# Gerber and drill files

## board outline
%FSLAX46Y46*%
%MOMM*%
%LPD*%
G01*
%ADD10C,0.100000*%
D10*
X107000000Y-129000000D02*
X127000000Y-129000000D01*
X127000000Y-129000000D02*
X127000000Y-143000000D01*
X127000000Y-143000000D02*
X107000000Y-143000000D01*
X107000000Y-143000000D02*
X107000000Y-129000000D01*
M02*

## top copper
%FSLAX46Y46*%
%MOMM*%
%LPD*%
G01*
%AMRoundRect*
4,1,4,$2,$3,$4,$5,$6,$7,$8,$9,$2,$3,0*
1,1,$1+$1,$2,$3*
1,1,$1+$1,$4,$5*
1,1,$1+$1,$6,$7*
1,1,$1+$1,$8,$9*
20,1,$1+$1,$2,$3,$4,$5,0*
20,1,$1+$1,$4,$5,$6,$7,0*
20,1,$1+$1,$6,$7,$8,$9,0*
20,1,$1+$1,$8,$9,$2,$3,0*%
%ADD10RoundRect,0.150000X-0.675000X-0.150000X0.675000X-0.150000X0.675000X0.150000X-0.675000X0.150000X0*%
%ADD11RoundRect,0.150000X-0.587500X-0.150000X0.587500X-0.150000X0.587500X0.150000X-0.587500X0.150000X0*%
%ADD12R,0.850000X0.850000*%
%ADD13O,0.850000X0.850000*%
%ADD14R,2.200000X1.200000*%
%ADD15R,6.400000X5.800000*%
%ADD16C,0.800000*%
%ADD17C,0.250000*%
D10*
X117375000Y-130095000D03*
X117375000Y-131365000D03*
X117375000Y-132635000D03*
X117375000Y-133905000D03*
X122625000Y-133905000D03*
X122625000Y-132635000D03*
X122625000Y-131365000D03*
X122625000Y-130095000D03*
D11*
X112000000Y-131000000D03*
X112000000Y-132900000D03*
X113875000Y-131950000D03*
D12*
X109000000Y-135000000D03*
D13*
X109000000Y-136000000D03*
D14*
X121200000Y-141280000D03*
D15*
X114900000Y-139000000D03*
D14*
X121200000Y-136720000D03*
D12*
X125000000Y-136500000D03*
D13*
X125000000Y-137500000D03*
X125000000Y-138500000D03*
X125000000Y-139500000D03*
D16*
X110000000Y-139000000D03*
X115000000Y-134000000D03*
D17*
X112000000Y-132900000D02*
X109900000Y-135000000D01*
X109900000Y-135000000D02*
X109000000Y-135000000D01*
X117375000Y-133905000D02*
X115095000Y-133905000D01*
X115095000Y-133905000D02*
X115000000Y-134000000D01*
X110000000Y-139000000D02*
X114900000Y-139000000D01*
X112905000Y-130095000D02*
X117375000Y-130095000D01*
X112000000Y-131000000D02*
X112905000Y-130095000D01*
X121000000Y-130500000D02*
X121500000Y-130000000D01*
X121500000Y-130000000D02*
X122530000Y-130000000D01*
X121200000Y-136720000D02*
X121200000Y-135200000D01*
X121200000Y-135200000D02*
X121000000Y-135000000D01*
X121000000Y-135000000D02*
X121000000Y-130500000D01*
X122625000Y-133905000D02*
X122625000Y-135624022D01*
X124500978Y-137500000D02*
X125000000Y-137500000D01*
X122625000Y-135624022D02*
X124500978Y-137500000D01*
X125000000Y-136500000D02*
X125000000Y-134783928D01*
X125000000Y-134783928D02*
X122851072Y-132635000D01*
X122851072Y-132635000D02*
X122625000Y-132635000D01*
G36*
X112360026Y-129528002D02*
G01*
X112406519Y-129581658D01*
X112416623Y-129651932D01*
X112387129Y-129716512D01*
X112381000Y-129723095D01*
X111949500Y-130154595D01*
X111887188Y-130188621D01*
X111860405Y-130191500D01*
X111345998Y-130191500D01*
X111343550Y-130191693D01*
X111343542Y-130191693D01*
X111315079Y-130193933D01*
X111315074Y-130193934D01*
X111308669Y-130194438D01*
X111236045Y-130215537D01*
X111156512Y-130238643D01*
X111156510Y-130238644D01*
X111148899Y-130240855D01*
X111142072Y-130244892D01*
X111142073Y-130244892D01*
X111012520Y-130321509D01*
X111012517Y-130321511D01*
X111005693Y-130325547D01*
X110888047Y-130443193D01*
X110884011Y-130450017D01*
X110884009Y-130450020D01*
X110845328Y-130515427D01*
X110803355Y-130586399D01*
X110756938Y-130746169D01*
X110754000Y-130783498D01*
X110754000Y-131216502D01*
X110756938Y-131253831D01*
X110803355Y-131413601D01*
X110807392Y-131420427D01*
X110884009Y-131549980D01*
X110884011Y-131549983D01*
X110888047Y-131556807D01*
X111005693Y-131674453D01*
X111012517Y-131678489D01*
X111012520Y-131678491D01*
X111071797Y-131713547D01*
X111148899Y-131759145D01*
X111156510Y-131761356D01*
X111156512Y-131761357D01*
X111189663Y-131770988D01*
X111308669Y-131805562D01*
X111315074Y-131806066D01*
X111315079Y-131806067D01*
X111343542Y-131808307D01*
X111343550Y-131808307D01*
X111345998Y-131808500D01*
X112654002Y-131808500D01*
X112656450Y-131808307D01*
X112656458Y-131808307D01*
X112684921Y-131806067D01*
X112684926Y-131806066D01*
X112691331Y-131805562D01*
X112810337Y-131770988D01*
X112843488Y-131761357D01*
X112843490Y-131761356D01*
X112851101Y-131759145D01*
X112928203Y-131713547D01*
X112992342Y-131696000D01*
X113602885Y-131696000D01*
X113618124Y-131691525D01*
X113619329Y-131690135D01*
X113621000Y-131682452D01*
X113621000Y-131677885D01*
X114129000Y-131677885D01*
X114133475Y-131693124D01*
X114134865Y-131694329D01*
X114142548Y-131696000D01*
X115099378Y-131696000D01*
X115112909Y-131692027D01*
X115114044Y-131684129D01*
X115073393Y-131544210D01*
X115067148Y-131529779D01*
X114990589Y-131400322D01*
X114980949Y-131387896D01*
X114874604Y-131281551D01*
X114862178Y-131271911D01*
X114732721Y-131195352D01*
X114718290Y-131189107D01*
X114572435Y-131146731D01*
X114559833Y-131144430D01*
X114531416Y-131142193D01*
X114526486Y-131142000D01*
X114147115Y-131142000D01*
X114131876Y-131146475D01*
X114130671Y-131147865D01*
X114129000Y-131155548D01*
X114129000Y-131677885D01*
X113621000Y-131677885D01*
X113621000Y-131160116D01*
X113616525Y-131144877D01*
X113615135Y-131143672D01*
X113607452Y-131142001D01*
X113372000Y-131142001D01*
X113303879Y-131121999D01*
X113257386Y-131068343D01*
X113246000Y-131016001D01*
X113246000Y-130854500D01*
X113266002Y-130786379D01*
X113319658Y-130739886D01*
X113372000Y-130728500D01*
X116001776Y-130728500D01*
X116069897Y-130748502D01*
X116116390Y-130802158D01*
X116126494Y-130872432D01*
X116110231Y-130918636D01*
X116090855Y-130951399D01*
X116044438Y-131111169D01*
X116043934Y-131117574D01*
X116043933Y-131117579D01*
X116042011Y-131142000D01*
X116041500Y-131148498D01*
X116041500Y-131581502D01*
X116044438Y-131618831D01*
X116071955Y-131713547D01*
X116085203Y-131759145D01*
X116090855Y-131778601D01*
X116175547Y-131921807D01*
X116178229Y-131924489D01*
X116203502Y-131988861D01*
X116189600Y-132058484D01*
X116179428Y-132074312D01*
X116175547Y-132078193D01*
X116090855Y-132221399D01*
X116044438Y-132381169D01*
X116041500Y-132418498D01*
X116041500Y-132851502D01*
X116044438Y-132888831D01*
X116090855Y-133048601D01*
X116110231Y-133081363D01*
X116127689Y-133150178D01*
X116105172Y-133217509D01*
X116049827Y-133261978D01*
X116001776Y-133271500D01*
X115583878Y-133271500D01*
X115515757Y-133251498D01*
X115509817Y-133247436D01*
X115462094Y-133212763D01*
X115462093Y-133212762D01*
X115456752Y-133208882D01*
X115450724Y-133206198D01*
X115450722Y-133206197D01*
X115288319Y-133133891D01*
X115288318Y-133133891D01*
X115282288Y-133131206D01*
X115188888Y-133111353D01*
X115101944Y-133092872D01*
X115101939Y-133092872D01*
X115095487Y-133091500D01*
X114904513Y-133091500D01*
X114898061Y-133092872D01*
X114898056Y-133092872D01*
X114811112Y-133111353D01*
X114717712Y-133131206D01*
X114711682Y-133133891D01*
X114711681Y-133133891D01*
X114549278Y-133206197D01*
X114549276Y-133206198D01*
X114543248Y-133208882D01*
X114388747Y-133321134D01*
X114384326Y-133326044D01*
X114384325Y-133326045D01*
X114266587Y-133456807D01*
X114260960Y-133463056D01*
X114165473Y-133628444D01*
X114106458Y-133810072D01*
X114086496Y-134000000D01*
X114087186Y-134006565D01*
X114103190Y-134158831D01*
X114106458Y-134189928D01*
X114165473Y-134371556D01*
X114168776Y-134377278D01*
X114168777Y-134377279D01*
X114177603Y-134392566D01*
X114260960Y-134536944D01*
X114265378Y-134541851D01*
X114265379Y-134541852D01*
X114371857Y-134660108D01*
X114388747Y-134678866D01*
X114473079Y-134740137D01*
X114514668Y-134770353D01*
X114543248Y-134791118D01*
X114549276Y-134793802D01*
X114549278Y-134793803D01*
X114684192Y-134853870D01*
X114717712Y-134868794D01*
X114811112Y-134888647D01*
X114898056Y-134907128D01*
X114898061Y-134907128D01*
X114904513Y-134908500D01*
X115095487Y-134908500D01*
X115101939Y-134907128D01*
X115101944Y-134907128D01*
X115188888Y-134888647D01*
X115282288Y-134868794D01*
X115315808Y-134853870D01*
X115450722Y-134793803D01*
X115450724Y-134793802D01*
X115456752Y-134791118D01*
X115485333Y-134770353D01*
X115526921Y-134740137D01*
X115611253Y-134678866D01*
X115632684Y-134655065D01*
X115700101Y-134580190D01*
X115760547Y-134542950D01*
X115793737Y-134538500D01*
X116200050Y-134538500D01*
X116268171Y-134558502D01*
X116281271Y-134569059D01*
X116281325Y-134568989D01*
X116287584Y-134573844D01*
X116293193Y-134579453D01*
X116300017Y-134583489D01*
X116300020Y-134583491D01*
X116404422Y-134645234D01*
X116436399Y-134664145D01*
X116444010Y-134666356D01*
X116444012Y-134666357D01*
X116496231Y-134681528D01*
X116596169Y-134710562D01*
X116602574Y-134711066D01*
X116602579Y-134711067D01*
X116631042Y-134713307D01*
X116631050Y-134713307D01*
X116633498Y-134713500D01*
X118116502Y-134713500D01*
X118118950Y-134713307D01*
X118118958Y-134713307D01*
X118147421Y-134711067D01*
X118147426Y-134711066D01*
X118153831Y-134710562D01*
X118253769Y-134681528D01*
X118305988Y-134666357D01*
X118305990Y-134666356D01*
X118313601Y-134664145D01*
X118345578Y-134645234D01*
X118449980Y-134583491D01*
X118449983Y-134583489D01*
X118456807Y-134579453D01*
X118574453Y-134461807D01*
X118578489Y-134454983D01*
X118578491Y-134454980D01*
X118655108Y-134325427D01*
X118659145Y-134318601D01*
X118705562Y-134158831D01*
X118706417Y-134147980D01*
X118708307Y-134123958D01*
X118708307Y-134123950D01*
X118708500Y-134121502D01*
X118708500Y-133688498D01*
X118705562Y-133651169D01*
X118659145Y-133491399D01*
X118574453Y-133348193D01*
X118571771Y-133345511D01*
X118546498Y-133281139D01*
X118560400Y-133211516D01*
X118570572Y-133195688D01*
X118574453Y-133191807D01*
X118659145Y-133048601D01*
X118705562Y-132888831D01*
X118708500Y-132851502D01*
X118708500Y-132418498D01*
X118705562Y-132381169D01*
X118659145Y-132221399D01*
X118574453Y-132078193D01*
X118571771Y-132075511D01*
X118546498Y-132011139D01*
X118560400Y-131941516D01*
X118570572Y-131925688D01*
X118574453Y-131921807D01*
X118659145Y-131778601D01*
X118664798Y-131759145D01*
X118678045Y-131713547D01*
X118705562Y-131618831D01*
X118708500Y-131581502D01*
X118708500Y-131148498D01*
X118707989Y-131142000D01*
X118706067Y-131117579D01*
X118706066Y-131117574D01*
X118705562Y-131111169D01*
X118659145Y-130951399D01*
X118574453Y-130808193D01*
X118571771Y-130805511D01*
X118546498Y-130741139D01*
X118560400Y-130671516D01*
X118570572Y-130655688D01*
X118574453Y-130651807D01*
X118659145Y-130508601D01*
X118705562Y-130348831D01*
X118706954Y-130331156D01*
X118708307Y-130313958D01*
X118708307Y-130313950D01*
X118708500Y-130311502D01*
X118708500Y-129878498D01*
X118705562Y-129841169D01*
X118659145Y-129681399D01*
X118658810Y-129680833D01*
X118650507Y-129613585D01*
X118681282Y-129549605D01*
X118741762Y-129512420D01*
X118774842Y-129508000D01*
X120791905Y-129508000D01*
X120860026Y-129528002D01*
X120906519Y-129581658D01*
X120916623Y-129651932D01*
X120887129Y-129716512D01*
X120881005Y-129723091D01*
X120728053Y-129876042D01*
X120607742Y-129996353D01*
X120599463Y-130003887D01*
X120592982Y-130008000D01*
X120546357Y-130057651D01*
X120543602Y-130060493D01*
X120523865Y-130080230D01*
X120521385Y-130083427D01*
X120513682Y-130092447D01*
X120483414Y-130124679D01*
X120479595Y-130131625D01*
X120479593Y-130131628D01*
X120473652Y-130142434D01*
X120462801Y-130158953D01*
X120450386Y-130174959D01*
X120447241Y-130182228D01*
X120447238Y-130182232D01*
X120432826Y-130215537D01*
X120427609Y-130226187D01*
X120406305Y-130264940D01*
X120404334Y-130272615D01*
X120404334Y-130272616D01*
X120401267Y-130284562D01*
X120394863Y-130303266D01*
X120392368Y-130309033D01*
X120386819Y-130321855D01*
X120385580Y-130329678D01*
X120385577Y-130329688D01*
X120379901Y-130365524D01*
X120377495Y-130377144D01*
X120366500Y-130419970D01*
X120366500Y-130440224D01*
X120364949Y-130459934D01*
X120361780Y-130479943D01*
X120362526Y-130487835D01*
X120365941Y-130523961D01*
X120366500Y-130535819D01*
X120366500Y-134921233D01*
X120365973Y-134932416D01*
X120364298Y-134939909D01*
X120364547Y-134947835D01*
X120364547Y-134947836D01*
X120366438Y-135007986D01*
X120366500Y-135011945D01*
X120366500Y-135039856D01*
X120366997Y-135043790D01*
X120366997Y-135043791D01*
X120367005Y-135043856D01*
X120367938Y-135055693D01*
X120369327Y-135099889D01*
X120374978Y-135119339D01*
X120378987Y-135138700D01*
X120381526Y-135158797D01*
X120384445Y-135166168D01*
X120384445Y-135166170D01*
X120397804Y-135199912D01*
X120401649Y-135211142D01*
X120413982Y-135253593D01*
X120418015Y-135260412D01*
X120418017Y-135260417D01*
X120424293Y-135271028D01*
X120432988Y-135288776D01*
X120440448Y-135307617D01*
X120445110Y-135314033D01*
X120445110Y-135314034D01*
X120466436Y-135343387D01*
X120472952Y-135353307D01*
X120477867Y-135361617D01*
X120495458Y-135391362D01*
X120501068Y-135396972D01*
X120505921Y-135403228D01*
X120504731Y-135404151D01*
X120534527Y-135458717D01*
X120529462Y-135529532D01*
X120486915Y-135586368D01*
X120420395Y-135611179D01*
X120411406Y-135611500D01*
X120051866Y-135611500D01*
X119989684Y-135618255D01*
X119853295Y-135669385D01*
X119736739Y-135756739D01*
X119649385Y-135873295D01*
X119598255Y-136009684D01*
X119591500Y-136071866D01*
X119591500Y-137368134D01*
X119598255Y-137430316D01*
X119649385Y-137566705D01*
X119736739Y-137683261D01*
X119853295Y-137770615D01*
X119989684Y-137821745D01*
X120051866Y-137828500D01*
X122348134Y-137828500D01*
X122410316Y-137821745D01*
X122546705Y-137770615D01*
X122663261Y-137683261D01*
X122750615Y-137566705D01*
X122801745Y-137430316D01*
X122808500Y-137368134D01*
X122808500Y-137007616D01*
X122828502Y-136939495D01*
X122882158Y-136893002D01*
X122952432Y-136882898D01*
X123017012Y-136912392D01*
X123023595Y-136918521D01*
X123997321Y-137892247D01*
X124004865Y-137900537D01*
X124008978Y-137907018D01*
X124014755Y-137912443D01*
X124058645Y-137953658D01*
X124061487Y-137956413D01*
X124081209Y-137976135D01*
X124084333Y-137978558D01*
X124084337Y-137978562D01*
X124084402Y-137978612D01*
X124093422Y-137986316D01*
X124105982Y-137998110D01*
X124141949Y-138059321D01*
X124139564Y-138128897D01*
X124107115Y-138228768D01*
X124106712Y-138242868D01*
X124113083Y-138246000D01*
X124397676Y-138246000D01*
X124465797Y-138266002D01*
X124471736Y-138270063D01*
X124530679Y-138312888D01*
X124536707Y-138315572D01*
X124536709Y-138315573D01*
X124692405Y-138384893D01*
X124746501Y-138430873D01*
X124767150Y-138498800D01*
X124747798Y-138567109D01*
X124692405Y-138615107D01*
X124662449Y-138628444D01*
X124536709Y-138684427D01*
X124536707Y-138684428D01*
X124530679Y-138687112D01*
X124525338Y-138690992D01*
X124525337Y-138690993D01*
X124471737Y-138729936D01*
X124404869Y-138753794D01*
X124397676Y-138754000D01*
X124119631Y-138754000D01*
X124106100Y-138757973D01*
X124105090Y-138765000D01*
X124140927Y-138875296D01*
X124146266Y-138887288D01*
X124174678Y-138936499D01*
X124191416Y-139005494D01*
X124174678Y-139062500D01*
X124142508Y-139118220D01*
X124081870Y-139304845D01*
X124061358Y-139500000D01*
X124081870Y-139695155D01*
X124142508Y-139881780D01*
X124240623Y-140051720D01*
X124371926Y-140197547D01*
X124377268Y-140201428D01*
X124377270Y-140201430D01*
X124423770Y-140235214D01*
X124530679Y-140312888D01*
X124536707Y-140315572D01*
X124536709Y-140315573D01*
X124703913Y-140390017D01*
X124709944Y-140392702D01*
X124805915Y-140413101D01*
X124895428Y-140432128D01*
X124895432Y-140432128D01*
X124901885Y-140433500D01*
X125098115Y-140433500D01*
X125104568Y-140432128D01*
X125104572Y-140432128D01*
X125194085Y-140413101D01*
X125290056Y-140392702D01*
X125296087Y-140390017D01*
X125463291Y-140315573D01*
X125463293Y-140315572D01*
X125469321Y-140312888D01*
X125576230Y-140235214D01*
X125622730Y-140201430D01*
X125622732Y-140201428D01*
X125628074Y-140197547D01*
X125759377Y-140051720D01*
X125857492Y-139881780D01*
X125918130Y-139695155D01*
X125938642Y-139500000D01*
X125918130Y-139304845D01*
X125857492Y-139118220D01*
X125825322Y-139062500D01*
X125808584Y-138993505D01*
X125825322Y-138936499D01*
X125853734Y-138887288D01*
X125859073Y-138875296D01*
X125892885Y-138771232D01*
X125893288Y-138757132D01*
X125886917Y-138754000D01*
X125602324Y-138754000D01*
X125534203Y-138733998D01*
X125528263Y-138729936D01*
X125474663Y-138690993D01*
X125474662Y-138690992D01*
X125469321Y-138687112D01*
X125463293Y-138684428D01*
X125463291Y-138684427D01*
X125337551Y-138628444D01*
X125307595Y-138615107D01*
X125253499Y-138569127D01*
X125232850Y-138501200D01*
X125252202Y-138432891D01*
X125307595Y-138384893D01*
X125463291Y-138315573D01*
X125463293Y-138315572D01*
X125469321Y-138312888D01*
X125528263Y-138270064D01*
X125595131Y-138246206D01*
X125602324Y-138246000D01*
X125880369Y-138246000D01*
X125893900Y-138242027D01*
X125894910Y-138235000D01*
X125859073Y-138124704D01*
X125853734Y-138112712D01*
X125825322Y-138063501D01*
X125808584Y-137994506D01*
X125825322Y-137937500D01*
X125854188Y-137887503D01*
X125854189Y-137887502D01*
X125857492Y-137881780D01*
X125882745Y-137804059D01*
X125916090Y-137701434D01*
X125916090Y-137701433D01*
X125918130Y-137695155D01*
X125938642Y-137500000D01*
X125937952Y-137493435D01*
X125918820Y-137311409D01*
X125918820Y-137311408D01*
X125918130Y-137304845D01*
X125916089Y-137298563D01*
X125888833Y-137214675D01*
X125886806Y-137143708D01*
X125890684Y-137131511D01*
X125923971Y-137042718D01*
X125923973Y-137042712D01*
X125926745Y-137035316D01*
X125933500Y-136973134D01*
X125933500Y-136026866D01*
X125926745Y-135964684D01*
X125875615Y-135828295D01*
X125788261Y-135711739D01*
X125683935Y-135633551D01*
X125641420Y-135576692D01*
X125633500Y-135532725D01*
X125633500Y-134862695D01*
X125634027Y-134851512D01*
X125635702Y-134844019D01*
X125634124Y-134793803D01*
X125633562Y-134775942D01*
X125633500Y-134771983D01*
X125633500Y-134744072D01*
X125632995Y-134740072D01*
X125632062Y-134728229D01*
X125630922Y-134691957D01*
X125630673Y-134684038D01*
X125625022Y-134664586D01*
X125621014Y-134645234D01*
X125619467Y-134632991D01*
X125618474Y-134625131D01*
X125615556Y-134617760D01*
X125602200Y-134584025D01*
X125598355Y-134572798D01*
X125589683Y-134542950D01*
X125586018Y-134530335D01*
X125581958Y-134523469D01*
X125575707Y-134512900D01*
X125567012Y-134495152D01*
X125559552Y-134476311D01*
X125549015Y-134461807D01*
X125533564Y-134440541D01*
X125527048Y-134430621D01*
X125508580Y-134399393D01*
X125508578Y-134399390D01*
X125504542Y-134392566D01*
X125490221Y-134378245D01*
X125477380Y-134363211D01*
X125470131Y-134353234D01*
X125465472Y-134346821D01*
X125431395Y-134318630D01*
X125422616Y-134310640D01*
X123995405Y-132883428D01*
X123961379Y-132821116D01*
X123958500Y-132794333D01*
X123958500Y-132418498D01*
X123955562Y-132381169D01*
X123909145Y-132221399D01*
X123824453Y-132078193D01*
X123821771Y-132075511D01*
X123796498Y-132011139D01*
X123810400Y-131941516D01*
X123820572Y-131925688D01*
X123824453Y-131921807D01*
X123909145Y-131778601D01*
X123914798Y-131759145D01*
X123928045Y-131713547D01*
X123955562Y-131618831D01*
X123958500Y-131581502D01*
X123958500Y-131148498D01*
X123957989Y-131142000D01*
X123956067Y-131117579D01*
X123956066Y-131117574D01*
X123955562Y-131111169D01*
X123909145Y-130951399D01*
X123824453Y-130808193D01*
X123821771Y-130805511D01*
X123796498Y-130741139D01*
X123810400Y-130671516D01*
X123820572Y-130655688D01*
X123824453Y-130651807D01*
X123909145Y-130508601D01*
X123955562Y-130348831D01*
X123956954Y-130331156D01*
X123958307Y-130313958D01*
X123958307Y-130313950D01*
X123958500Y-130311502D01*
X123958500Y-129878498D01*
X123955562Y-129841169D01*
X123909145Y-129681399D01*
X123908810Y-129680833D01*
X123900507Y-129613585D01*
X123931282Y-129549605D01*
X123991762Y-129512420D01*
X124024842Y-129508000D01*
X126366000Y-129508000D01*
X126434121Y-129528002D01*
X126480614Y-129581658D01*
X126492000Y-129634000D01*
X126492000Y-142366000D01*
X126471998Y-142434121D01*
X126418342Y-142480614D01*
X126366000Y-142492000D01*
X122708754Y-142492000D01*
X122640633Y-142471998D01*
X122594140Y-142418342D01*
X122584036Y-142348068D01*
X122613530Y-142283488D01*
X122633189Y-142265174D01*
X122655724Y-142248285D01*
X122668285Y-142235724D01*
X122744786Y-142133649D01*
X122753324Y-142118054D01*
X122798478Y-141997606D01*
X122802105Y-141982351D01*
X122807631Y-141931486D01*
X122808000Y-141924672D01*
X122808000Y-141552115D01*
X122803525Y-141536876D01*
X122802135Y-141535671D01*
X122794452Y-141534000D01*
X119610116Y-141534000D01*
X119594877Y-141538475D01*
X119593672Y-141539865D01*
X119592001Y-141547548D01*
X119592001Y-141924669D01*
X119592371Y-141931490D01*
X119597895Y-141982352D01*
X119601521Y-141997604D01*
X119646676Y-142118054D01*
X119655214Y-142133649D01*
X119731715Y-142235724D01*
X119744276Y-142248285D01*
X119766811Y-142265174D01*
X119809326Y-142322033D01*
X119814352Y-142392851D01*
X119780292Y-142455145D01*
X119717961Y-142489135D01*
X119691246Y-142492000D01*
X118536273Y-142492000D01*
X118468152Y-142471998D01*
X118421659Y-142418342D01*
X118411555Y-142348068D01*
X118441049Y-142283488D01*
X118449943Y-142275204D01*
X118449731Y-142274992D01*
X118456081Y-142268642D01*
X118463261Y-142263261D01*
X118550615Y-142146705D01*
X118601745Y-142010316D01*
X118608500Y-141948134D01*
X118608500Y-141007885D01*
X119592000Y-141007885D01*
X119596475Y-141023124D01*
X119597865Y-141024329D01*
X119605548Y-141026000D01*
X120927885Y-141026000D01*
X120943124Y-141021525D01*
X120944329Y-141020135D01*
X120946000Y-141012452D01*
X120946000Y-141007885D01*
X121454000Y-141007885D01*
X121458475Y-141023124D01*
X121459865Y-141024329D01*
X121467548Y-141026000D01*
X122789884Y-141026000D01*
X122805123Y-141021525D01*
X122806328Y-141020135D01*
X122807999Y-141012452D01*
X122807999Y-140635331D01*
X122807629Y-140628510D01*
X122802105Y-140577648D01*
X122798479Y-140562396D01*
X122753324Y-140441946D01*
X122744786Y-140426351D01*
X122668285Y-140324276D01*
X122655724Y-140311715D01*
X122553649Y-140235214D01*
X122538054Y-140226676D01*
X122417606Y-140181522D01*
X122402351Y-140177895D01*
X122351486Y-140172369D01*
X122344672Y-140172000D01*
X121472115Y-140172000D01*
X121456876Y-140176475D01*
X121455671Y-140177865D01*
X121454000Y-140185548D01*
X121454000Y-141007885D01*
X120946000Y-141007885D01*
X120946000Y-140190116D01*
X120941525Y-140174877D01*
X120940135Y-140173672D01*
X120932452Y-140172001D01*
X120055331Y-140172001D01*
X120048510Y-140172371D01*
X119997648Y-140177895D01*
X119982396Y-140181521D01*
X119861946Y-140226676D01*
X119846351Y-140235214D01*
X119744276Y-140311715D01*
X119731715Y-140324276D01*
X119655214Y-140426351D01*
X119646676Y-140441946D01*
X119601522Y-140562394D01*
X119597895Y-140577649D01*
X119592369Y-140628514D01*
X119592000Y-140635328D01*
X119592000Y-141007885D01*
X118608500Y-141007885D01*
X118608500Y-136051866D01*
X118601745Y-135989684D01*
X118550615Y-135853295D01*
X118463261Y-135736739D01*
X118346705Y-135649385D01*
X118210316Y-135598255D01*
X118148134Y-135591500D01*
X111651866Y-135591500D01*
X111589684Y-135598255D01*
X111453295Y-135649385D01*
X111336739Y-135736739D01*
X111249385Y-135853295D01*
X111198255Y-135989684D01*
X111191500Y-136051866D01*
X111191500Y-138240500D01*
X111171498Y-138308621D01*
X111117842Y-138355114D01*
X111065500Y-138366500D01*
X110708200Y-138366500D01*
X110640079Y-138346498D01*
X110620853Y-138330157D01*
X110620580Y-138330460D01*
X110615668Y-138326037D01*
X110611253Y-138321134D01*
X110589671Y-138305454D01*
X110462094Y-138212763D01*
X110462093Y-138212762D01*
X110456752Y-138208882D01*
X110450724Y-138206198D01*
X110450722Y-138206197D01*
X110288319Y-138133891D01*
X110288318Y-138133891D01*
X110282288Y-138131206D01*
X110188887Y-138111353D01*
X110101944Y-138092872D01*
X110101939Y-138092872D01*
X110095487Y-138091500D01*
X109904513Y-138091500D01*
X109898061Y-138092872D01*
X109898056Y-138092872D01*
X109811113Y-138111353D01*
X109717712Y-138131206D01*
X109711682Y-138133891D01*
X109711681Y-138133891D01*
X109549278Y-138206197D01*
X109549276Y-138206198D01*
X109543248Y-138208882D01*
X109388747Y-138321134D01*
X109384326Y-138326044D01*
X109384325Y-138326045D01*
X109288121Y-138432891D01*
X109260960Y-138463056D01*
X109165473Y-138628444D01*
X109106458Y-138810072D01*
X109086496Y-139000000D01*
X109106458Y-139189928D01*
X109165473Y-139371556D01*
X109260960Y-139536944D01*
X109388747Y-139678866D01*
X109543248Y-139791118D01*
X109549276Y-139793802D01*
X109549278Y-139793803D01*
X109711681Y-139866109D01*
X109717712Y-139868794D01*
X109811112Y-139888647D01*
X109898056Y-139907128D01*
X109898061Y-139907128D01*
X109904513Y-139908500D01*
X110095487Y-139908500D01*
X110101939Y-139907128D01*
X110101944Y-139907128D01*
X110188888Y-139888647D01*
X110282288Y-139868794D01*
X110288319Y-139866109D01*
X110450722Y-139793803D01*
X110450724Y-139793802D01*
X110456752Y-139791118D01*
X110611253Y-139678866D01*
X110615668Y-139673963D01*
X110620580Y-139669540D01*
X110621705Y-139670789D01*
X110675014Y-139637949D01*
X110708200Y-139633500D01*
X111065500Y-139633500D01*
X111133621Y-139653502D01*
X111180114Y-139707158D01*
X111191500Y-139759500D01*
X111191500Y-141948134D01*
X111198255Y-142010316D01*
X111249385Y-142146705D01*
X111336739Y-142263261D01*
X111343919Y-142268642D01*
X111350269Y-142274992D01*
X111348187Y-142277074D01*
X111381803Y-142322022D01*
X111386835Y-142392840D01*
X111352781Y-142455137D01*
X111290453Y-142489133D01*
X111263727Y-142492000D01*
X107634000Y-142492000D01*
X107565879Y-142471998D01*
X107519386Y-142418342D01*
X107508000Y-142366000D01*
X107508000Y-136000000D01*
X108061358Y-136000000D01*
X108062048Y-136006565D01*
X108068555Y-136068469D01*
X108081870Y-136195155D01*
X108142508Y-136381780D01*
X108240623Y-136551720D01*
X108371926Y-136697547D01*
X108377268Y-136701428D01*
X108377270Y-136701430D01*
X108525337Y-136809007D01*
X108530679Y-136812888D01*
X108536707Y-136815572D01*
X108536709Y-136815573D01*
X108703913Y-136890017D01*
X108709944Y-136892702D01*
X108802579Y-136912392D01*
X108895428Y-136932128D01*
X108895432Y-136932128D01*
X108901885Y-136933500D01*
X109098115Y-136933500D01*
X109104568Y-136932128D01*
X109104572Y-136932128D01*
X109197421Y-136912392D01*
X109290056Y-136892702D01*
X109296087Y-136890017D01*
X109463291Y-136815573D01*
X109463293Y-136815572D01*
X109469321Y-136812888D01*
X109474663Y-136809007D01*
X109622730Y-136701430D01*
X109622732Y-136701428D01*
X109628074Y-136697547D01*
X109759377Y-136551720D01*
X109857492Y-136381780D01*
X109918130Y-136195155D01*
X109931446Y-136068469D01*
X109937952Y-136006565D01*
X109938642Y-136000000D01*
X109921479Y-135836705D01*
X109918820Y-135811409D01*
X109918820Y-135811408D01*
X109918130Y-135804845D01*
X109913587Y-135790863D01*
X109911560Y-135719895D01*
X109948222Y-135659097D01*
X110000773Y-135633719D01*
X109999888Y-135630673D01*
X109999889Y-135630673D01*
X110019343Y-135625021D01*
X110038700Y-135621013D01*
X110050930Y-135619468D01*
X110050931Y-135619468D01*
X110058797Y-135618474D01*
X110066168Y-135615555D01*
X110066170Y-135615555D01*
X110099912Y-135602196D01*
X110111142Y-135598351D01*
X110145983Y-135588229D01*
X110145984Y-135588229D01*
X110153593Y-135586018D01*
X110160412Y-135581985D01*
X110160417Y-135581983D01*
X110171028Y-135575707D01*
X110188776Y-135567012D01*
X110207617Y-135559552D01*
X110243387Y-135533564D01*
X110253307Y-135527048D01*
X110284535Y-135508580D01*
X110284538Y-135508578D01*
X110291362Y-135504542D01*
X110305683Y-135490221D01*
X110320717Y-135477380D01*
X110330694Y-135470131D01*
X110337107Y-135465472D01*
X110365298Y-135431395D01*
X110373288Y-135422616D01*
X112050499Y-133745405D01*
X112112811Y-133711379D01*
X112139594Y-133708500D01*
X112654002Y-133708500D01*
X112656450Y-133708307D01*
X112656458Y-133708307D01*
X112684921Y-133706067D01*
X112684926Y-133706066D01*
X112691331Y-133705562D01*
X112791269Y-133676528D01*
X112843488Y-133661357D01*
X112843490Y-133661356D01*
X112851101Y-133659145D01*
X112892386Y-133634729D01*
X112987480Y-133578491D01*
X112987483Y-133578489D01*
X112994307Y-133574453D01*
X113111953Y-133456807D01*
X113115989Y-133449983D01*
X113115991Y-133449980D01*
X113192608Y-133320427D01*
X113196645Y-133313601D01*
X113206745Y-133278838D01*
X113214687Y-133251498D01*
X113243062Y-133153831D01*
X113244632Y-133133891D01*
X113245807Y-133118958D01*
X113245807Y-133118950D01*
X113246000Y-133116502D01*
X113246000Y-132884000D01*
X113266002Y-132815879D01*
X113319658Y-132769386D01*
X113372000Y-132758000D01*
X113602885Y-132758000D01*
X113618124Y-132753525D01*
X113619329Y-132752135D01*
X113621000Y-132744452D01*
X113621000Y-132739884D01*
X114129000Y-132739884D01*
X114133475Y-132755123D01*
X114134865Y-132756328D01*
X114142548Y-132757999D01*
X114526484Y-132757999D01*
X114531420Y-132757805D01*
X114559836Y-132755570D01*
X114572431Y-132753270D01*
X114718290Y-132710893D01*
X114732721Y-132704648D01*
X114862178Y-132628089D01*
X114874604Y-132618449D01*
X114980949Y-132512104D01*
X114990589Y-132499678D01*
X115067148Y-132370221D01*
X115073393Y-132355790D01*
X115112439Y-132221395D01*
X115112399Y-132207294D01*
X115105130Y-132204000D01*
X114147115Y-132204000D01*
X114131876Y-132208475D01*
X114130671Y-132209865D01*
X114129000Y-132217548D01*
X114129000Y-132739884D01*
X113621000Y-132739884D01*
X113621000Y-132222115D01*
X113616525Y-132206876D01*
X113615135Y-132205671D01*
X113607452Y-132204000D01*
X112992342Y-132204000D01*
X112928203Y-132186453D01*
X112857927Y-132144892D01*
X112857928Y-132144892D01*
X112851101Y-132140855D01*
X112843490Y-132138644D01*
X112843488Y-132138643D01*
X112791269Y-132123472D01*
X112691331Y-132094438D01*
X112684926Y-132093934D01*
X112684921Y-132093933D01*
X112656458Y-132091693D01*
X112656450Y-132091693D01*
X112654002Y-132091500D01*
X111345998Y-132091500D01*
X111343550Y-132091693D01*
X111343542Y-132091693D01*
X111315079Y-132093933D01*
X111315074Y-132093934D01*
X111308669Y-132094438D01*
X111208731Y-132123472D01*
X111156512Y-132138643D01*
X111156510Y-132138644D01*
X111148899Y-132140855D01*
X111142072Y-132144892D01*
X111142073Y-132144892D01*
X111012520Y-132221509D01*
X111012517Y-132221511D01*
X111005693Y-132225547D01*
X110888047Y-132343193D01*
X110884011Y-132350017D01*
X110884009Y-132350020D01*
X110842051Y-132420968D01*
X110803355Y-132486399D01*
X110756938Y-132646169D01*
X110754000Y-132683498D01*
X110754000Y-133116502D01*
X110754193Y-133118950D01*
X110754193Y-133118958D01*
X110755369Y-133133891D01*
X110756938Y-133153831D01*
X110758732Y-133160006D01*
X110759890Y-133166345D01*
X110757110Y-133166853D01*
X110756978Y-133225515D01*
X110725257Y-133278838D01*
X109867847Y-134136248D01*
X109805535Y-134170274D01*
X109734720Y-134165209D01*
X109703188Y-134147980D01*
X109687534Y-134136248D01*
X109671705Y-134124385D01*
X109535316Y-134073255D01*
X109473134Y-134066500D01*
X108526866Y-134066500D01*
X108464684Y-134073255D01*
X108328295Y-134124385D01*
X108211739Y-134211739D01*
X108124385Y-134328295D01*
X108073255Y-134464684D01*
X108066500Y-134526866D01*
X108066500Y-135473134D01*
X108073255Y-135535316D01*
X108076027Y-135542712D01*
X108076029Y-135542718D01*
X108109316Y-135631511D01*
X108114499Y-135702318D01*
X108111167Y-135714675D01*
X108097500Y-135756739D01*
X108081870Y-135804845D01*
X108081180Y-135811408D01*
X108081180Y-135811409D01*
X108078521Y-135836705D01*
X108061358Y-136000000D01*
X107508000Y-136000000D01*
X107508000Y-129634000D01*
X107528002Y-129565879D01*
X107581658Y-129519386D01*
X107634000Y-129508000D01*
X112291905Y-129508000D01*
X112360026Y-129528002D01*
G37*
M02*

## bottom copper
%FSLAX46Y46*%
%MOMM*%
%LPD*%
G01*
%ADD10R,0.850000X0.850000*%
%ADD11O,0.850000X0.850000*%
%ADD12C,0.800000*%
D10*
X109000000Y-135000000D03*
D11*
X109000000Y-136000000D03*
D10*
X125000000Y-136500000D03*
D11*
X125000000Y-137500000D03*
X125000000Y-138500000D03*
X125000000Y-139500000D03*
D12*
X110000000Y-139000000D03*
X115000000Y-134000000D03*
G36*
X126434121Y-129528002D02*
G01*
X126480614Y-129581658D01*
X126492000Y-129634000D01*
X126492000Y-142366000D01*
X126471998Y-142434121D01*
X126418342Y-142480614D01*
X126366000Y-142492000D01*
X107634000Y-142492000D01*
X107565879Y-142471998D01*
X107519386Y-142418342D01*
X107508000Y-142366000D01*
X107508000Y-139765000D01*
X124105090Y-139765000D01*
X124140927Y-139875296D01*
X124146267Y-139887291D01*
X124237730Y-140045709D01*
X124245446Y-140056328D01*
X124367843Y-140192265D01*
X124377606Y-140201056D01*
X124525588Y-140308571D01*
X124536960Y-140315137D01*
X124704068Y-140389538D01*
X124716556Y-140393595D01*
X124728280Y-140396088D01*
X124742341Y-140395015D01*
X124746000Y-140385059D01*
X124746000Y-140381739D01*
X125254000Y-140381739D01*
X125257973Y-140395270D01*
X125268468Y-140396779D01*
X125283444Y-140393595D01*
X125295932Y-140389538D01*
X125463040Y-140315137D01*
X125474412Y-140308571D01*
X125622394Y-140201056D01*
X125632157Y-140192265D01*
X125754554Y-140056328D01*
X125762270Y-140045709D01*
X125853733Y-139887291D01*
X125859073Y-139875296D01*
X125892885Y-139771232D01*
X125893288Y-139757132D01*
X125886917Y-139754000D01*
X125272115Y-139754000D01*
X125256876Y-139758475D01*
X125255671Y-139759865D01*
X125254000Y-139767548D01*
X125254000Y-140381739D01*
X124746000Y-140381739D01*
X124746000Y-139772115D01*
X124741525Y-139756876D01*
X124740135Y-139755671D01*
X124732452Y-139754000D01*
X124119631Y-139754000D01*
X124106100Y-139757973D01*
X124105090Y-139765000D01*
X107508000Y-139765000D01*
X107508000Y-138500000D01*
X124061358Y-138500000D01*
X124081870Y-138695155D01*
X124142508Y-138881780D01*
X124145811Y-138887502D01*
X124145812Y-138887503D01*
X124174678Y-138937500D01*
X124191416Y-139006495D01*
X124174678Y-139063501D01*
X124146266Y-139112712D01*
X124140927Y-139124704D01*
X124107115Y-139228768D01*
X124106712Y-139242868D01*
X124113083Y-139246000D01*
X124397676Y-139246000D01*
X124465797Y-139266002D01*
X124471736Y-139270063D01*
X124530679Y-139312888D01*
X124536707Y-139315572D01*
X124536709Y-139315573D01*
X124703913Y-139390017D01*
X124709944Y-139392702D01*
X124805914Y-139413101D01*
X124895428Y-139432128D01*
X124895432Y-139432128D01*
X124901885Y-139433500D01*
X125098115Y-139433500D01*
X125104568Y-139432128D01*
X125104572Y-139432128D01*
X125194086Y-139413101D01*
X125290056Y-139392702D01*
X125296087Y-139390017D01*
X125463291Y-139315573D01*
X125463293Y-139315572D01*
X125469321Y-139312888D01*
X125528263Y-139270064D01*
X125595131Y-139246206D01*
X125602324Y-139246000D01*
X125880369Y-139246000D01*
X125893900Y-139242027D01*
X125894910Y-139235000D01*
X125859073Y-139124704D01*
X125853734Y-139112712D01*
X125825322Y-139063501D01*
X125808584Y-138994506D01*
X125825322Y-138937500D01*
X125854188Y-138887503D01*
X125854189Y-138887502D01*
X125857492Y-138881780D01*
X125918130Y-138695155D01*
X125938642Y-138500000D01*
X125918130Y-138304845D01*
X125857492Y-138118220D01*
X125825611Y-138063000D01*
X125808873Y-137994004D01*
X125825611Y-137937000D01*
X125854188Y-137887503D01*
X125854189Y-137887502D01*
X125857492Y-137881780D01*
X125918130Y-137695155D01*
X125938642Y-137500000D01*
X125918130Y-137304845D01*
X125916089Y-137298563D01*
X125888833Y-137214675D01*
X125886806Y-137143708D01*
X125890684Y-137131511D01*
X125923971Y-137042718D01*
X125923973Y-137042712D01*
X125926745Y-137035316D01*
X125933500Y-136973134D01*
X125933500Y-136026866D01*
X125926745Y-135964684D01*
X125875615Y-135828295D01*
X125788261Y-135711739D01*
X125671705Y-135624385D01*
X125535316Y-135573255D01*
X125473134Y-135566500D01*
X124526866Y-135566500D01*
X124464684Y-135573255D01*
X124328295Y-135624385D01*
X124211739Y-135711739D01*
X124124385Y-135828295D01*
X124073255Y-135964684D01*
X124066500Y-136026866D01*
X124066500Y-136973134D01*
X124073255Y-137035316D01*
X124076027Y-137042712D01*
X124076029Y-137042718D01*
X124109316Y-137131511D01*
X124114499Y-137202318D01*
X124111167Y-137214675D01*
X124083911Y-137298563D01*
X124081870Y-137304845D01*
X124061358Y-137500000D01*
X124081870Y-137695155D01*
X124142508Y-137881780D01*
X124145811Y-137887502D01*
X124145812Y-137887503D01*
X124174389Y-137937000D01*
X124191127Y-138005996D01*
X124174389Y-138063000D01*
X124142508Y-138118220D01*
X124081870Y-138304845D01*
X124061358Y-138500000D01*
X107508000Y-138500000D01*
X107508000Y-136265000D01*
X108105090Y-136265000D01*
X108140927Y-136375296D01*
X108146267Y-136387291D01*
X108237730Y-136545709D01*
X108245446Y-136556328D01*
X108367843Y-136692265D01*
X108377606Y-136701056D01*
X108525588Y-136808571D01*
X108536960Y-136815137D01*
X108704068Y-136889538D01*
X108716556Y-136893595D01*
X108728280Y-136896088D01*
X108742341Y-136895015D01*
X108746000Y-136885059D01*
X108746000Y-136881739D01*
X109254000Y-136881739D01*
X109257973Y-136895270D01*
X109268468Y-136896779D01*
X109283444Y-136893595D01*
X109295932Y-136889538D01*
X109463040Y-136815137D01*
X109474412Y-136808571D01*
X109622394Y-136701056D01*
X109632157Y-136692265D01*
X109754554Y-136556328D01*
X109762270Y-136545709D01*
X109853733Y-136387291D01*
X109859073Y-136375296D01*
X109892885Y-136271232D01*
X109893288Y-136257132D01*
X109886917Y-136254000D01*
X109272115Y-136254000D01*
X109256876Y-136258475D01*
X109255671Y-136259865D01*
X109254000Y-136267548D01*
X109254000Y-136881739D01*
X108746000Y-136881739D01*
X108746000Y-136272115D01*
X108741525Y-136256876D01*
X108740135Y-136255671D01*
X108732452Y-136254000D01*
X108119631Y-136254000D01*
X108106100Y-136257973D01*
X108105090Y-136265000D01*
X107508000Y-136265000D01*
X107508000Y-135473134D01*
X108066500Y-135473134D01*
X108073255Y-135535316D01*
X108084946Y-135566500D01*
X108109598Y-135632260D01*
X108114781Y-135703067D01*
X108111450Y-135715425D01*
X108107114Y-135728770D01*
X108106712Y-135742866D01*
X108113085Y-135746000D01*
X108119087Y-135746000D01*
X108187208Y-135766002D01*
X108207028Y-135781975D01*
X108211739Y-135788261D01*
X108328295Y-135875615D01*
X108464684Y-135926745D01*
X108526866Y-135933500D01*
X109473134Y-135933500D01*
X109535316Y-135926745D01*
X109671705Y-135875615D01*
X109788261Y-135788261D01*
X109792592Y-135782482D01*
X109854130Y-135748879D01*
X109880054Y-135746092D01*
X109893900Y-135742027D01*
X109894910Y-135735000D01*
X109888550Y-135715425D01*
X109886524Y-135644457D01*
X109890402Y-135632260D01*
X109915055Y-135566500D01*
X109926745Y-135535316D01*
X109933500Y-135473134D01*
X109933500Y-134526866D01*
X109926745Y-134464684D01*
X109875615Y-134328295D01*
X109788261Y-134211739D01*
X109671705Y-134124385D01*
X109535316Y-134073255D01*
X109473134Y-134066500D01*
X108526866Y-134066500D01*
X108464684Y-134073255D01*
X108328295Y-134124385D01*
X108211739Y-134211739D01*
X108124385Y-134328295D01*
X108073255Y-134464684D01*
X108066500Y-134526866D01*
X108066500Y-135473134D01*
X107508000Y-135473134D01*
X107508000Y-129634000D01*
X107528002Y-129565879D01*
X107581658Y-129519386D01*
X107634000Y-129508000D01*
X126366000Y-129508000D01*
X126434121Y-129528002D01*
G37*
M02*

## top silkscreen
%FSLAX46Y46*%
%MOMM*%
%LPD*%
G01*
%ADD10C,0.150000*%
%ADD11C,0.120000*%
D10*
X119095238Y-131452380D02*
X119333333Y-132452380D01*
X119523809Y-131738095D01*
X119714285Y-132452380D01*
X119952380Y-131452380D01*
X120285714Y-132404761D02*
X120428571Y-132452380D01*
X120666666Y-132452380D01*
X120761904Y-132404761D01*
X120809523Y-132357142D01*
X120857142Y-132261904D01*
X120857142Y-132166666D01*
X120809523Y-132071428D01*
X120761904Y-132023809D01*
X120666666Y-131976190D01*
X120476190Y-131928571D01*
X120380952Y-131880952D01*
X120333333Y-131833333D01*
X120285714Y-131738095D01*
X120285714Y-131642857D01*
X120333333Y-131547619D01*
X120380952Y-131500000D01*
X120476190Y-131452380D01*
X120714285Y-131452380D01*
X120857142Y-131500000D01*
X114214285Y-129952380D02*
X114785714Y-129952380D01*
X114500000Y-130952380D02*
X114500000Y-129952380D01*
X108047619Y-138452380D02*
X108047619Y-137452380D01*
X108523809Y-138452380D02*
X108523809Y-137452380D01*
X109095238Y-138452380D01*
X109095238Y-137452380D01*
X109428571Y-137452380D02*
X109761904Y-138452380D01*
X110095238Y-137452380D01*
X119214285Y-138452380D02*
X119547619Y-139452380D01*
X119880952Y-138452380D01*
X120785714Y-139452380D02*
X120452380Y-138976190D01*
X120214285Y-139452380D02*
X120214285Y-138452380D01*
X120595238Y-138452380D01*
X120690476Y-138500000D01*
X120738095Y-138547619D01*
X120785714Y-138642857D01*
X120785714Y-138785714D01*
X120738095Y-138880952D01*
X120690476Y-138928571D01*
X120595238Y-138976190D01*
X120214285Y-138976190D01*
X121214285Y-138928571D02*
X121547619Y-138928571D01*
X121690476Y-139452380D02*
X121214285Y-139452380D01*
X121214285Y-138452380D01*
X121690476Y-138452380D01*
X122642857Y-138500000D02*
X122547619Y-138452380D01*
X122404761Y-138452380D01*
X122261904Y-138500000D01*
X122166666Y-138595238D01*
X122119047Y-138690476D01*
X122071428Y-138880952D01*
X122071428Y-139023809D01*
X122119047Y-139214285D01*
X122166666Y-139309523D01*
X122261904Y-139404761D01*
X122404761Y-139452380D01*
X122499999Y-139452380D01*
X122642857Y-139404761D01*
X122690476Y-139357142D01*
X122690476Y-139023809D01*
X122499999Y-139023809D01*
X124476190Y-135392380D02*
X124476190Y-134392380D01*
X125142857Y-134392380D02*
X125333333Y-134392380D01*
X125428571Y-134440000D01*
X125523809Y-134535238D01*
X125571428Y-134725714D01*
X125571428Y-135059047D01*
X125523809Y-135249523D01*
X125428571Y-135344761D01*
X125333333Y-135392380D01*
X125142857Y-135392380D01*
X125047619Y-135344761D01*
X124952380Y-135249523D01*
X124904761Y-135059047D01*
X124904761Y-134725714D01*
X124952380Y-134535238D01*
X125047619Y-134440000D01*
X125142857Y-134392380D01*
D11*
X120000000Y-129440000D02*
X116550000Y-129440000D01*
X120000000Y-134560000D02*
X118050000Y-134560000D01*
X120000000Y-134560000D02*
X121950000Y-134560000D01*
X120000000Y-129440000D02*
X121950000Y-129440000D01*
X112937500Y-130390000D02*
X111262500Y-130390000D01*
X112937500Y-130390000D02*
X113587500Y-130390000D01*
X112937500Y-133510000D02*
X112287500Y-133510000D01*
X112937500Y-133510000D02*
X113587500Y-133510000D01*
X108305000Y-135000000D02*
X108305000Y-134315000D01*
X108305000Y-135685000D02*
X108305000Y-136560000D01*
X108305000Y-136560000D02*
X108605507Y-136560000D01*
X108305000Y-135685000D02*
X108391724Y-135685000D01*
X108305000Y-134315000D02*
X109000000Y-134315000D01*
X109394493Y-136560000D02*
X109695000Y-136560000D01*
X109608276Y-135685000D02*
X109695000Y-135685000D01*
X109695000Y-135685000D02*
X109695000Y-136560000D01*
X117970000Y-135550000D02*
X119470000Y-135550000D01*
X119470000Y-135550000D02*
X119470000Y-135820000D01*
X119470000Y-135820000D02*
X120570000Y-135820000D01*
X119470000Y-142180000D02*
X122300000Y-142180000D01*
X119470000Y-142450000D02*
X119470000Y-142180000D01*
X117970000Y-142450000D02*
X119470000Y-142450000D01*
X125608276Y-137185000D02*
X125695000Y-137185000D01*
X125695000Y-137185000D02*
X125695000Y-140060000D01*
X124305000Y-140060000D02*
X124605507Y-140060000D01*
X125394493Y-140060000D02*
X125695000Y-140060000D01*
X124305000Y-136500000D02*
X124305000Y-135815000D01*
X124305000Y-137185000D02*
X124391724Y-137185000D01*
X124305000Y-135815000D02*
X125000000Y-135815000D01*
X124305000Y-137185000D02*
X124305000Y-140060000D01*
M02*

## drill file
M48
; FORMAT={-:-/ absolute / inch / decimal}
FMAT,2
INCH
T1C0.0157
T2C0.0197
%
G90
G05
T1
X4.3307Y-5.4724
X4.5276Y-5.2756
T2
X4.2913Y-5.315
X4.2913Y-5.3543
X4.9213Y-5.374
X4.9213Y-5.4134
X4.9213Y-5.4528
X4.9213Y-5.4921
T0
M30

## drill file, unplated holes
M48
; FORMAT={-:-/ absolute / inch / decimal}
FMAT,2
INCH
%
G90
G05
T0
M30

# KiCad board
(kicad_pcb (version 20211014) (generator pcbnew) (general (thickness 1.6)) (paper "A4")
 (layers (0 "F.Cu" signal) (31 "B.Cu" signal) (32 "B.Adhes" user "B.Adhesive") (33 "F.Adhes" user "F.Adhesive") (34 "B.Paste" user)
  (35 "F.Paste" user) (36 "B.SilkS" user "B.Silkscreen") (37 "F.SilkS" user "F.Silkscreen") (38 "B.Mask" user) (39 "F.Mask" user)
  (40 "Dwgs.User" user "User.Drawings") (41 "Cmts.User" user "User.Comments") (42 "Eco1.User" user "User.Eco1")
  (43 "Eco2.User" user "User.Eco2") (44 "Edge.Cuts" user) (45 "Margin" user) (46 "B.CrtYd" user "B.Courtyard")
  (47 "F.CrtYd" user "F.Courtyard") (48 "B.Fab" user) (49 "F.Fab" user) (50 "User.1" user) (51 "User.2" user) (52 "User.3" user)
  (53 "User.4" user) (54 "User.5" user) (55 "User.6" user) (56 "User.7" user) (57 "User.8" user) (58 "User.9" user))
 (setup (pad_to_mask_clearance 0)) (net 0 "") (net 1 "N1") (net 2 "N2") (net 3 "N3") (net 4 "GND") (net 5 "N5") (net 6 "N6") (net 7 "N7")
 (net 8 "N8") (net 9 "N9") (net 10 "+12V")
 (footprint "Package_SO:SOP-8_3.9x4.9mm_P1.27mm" (layer "F.Cu") (at 120 132)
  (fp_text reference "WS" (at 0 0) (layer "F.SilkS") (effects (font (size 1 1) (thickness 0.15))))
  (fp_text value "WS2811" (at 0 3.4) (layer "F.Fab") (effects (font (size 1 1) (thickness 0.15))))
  (fp_line (start 0 -2.56) (end -3.45 -2.56) (layer "F.SilkS") (width 0.12))
  (fp_line (start 0 2.56) (end -1.95 2.56) (layer "F.SilkS") (width 0.12))
  (fp_line (start 0 2.56) (end 1.95 2.56) (layer "F.SilkS") (width 0.12))
  (fp_line (start 0 -2.56) (end 1.95 -2.56) (layer "F.SilkS") (width 0.12))
  (pad "1" smd roundrect (at -2.625 -1.905) (size 1.65 0.6) (layers "F.Cu" "F.Paste" "F.Mask") (roundrect_rratio 0.25) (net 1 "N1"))
  (pad "2" smd roundrect (at -2.625 -0.635) (size 1.65 0.6) (layers "F.Cu" "F.Paste" "F.Mask") (roundrect_rratio 0.25) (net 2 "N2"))
  (pad "3" smd roundrect (at -2.625 0.635) (size 1.65 0.6) (layers "F.Cu" "F.Paste" "F.Mask") (roundrect_rratio 0.25) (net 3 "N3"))
  (pad "4" smd roundrect (at -2.625 1.905) (size 1.65 0.6) (layers "F.Cu" "F.Paste" "F.Mask") (roundrect_rratio 0.25) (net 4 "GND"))
  (pad "5" smd roundrect (at 2.625 1.905) (size 1.65 0.6) (layers "F.Cu" "F.Paste" "F.Mask") (roundrect_rratio 0.25) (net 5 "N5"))
  (pad "6" smd roundrect (at 2.625 0.635) (size 1.65 0.6) (layers "F.Cu" "F.Paste" "F.Mask") (roundrect_rratio 0.25) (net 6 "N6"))
  (pad "7" smd roundrect (at 2.625 -0.635) (size 1.65 0.6) (layers "F.Cu" "F.Paste" "F.Mask") (roundrect_rratio 0.25) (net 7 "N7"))
  (pad "8" smd roundrect (at 2.625 -1.905) (size 1.65 0.6) (layers "F.Cu" "F.Paste" "F.Mask") (roundrect_rratio 0.25) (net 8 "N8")))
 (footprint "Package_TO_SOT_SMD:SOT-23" (layer "F.Cu") (at 112.9375 131.95)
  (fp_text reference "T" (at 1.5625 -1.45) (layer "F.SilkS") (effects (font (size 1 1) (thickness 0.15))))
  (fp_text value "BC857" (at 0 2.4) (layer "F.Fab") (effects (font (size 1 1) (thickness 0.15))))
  (fp_line (start 0 -1.56) (end -1.675 -1.56) (layer "F.SilkS") (width 0.12))
  (fp_line (start 0 -1.56) (end 0.65 -1.56) (layer "F.SilkS") (width 0.12))
  (fp_line (start 0 1.56) (end -0.65 1.56) (layer "F.SilkS") (width 0.12))
  (fp_line (start 0 1.56) (end 0.65 1.56) (layer "F.SilkS") (width 0.12))
  (pad "1" smd roundrect (at -0.9375 -0.95) (size 1.475 0.6) (layers "F.Cu" "F.Paste" "F.Mask") (roundrect_rratio 0.25) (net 1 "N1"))
  (pad "2" smd roundrect (at -0.9375 0.95) (size 1.475 0.6) (layers "F.Cu" "F.Paste" "F.Mask") (roundrect_rratio 0.25) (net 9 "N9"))
  (pad "3" smd roundrect (at 0.9375 0) (size 1.475 0.6) (layers "F.Cu" "F.Paste" "F.Mask") (roundrect_rratio 0.25) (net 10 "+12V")))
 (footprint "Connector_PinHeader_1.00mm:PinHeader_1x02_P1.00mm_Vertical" (layer "F.Cu") (at 109 135)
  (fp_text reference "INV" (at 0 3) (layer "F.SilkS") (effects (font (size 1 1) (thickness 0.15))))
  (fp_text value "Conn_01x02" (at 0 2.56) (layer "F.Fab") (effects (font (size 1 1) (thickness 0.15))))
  (fp_line (start -0.695 0) (end -0.695 -0.685) (layer "F.SilkS") (width 0.12))
  (fp_line (start -0.695 0.685) (end -0.695 1.56) (layer "F.SilkS") (width 0.12))
  (fp_line (start -0.695 1.56) (end -0.394493 1.56) (layer "F.SilkS") (width 0.12))
  (fp_line (start -0.695 0.685) (end -0.608276 0.685) (layer "F.SilkS") (width 0.12))
  (fp_line (start -0.695 -0.685) (end 0 -0.685) (layer "F.SilkS") (width 0.12))
  (fp_line (start 0.394493 1.56) (end 0.695 1.56) (layer "F.SilkS") (width 0.12))
  (fp_line (start 0.608276 0.685) (end 0.695 0.685) (layer "F.SilkS") (width 0.12))
  (fp_line (start 0.695 0.685) (end 0.695 1.56) (layer "F.SilkS") (width 0.12))
  (pad "1" thru_hole rect (at 0 0) (size 0.85 0.85) (drill 0.5) (layers *.Cu *.Mask) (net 9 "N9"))
  (pad "2" thru_hole oval (at 0 1) (size 0.85 0.85) (drill 0.5) (layers *.Cu *.Mask) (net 4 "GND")))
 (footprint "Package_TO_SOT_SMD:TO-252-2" (layer "F.Cu") (at 117 139 180)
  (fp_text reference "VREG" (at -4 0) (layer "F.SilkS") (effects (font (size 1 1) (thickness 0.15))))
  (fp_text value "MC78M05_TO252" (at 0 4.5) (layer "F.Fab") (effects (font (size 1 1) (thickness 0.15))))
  (fp_line (start -0.97 3.45) (end -2.47 3.45) (layer "F.SilkS") (width 0.12))
  (fp_line (start -2.47 3.45) (end -2.47 3.18) (layer "F.SilkS") (width 0.12))
  (fp_line (start -2.47 3.18) (end -3.57 3.18) (layer "F.SilkS") (width 0.12))
  (fp_line (start -2.47 -3.18) (end -5.3 -3.18) (layer "F.SilkS") (width 0.12))
  (fp_line (start -2.47 -3.45) (end -2.47 -3.18) (layer "F.SilkS") (width 0.12))
  (fp_line (start -0.97 -3.45) (end -2.47 -3.45) (layer "F.SilkS") (width 0.12))
  (pad "" smd rect (at 0.425 -1.525 180) (size 3.05 2.75) (layers "F.Paste"))
  (pad "" smd rect (at 3.775 1.525 180) (size 3.05 2.75) (layers "F.Paste"))
  (pad "" smd rect (at 3.775 -1.525 180) (size 3.05 2.75) (layers "F.Paste"))
  (pad "" smd rect (at 0.425 1.525 180) (size 3.05 2.75) (layers "F.Paste"))
  (pad "1" smd rect (at -4.2 -2.28 180) (size 2.2 1.2) (layers "F.Cu" "F.Paste" "F.Mask") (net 10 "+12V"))
  (pad "2" smd rect (at 2.1 0 180) (size 6.4 5.8) (layers "F.Cu" "F.Mask") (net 4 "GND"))
  (pad "3" smd rect (at -4.2 2.28 180) (size 2.2 1.2) (layers "F.Cu" "F.Paste" "F.Mask") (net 8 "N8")))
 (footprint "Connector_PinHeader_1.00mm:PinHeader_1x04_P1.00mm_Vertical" (layer "F.Cu") (at 125 136.5)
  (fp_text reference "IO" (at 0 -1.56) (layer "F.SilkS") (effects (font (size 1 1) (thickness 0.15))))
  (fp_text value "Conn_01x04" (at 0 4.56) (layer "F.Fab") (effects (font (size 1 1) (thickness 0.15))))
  (fp_line (start 0.608276 0.685) (end 0.695 0.685) (layer "F.SilkS") (width 0.12))
  (fp_line (start 0.695 0.685) (end 0.695 3.56) (layer "F.SilkS") (width 0.12))
  (fp_line (start -0.695 3.56) (end -0.394493 3.56) (layer "F.SilkS") (width 0.12))
  (fp_line (start 0.394493 3.56) (end 0.695 3.56) (layer "F.SilkS") (width 0.12))
  (fp_line (start -0.695 0) (end -0.695 -0.685) (layer "F.SilkS") (width 0.12))
  (fp_line (start -0.695 0.685) (end -0.608276 0.685) (layer "F.SilkS") (width 0.12))
  (fp_line (start -0.695 -0.685) (end 0 -0.685) (layer "F.SilkS") (width 0.12))
  (fp_line (start -0.695 0.685) (end -0.695 3.56) (layer "F.SilkS") (width 0.12))
  (pad "1" thru_hole rect (at 0 0) (size 0.85 0.85) (drill 0.5) (layers *.Cu *.Mask) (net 6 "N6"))
  (pad "2" thru_hole oval (at 0 1) (size 0.85 0.85) (drill 0.5) (layers *.Cu *.Mask) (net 5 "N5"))
  (pad "3" thru_hole oval (at 0 2) (size 0.85 0.85) (drill 0.5) (layers *.Cu *.Mask) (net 10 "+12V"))
  (pad "4" thru_hole oval (at 0 3) (size 0.85 0.85) (drill 0.5) (layers *.Cu *.Mask) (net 4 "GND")))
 (gr_rect (start 107 129) (end 127 143) (layer "Edge.Cuts") (width 0.1) (fill none))
 (segment (start 109.9 135) (end 109 135) (width 0.25) (layer "F.Cu") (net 9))
 (segment (start 112 132.9) (end 109.9 135) (width 0.25) (layer "F.Cu") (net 9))
 (segment (start 117.375 133.905) (end 115.095 133.905) (width 0.25) (layer "F.Cu") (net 4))
 (segment (start 110 139) (end 114.9 139) (width 0.25) (layer "F.Cu") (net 4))
 (segment (start 115.095 133.905) (end 115 134) (width 0.25) (layer "F.Cu") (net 4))
 (via (at 110 139) (size 0.8) (drill 0.4) (layers "F.Cu" "B.Cu") (free) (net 4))
 (via (at 115 134) (size 0.8) (drill 0.4) (layers "F.Cu" "B.Cu") (free) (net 4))
 (segment (start 112.905 130.095) (end 117.375 130.095) (width 0.25) (layer "F.Cu") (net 1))
 (segment (start 112 131) (end 112.905 130.095) (width 0.25) (layer "F.Cu") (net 1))
 (segment (start 121 130.5) (end 121.5 130) (width 0.25) (layer "F.Cu") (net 8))
 (segment (start 121.5 130) (end 122.53 130) (width 0.25) (layer "F.Cu") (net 8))
 (segment (start 121.2 136.72) (end 121.2 135.2) (width 0.25) (layer "F.Cu") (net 8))
 (segment (start 121.2 135.2) (end 121 135) (width 0.25) (layer "F.Cu") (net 8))
 (segment (start 121 135) (end 121 130.5) (width 0.25) (layer "F.Cu") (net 8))
 (segment (start 122.625 133.905) (end 122.625 135.624022) (width 0.25) (layer "F.Cu") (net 5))
 (segment (start 124.500978 137.5) (end 125 137.5) (width 0.25) (layer "F.Cu") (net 5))
 (segment (start 122.625 135.624022) (end 124.500978 137.5) (width 0.25) (layer "F.Cu") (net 5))
 (segment (start 125 136.5) (end 125 134.783928) (width 0.25) (layer "F.Cu") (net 6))
 (segment (start 125 134.783928) (end 122.851072 132.635) (width 0.25) (layer "F.Cu") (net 6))
 (segment (start 122.851072 132.635) (end 122.625 132.635) (width 0.25) (layer "F.Cu") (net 6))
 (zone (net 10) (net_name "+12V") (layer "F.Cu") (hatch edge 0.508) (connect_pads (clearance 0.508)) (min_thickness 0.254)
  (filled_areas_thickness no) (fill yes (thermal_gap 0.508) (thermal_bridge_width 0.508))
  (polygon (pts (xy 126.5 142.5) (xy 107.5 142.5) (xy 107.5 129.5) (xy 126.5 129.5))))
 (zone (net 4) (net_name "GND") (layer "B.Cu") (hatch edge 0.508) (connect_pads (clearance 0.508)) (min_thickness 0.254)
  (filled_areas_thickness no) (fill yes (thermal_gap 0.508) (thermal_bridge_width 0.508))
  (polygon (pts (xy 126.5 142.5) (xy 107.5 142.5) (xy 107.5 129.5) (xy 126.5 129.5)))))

